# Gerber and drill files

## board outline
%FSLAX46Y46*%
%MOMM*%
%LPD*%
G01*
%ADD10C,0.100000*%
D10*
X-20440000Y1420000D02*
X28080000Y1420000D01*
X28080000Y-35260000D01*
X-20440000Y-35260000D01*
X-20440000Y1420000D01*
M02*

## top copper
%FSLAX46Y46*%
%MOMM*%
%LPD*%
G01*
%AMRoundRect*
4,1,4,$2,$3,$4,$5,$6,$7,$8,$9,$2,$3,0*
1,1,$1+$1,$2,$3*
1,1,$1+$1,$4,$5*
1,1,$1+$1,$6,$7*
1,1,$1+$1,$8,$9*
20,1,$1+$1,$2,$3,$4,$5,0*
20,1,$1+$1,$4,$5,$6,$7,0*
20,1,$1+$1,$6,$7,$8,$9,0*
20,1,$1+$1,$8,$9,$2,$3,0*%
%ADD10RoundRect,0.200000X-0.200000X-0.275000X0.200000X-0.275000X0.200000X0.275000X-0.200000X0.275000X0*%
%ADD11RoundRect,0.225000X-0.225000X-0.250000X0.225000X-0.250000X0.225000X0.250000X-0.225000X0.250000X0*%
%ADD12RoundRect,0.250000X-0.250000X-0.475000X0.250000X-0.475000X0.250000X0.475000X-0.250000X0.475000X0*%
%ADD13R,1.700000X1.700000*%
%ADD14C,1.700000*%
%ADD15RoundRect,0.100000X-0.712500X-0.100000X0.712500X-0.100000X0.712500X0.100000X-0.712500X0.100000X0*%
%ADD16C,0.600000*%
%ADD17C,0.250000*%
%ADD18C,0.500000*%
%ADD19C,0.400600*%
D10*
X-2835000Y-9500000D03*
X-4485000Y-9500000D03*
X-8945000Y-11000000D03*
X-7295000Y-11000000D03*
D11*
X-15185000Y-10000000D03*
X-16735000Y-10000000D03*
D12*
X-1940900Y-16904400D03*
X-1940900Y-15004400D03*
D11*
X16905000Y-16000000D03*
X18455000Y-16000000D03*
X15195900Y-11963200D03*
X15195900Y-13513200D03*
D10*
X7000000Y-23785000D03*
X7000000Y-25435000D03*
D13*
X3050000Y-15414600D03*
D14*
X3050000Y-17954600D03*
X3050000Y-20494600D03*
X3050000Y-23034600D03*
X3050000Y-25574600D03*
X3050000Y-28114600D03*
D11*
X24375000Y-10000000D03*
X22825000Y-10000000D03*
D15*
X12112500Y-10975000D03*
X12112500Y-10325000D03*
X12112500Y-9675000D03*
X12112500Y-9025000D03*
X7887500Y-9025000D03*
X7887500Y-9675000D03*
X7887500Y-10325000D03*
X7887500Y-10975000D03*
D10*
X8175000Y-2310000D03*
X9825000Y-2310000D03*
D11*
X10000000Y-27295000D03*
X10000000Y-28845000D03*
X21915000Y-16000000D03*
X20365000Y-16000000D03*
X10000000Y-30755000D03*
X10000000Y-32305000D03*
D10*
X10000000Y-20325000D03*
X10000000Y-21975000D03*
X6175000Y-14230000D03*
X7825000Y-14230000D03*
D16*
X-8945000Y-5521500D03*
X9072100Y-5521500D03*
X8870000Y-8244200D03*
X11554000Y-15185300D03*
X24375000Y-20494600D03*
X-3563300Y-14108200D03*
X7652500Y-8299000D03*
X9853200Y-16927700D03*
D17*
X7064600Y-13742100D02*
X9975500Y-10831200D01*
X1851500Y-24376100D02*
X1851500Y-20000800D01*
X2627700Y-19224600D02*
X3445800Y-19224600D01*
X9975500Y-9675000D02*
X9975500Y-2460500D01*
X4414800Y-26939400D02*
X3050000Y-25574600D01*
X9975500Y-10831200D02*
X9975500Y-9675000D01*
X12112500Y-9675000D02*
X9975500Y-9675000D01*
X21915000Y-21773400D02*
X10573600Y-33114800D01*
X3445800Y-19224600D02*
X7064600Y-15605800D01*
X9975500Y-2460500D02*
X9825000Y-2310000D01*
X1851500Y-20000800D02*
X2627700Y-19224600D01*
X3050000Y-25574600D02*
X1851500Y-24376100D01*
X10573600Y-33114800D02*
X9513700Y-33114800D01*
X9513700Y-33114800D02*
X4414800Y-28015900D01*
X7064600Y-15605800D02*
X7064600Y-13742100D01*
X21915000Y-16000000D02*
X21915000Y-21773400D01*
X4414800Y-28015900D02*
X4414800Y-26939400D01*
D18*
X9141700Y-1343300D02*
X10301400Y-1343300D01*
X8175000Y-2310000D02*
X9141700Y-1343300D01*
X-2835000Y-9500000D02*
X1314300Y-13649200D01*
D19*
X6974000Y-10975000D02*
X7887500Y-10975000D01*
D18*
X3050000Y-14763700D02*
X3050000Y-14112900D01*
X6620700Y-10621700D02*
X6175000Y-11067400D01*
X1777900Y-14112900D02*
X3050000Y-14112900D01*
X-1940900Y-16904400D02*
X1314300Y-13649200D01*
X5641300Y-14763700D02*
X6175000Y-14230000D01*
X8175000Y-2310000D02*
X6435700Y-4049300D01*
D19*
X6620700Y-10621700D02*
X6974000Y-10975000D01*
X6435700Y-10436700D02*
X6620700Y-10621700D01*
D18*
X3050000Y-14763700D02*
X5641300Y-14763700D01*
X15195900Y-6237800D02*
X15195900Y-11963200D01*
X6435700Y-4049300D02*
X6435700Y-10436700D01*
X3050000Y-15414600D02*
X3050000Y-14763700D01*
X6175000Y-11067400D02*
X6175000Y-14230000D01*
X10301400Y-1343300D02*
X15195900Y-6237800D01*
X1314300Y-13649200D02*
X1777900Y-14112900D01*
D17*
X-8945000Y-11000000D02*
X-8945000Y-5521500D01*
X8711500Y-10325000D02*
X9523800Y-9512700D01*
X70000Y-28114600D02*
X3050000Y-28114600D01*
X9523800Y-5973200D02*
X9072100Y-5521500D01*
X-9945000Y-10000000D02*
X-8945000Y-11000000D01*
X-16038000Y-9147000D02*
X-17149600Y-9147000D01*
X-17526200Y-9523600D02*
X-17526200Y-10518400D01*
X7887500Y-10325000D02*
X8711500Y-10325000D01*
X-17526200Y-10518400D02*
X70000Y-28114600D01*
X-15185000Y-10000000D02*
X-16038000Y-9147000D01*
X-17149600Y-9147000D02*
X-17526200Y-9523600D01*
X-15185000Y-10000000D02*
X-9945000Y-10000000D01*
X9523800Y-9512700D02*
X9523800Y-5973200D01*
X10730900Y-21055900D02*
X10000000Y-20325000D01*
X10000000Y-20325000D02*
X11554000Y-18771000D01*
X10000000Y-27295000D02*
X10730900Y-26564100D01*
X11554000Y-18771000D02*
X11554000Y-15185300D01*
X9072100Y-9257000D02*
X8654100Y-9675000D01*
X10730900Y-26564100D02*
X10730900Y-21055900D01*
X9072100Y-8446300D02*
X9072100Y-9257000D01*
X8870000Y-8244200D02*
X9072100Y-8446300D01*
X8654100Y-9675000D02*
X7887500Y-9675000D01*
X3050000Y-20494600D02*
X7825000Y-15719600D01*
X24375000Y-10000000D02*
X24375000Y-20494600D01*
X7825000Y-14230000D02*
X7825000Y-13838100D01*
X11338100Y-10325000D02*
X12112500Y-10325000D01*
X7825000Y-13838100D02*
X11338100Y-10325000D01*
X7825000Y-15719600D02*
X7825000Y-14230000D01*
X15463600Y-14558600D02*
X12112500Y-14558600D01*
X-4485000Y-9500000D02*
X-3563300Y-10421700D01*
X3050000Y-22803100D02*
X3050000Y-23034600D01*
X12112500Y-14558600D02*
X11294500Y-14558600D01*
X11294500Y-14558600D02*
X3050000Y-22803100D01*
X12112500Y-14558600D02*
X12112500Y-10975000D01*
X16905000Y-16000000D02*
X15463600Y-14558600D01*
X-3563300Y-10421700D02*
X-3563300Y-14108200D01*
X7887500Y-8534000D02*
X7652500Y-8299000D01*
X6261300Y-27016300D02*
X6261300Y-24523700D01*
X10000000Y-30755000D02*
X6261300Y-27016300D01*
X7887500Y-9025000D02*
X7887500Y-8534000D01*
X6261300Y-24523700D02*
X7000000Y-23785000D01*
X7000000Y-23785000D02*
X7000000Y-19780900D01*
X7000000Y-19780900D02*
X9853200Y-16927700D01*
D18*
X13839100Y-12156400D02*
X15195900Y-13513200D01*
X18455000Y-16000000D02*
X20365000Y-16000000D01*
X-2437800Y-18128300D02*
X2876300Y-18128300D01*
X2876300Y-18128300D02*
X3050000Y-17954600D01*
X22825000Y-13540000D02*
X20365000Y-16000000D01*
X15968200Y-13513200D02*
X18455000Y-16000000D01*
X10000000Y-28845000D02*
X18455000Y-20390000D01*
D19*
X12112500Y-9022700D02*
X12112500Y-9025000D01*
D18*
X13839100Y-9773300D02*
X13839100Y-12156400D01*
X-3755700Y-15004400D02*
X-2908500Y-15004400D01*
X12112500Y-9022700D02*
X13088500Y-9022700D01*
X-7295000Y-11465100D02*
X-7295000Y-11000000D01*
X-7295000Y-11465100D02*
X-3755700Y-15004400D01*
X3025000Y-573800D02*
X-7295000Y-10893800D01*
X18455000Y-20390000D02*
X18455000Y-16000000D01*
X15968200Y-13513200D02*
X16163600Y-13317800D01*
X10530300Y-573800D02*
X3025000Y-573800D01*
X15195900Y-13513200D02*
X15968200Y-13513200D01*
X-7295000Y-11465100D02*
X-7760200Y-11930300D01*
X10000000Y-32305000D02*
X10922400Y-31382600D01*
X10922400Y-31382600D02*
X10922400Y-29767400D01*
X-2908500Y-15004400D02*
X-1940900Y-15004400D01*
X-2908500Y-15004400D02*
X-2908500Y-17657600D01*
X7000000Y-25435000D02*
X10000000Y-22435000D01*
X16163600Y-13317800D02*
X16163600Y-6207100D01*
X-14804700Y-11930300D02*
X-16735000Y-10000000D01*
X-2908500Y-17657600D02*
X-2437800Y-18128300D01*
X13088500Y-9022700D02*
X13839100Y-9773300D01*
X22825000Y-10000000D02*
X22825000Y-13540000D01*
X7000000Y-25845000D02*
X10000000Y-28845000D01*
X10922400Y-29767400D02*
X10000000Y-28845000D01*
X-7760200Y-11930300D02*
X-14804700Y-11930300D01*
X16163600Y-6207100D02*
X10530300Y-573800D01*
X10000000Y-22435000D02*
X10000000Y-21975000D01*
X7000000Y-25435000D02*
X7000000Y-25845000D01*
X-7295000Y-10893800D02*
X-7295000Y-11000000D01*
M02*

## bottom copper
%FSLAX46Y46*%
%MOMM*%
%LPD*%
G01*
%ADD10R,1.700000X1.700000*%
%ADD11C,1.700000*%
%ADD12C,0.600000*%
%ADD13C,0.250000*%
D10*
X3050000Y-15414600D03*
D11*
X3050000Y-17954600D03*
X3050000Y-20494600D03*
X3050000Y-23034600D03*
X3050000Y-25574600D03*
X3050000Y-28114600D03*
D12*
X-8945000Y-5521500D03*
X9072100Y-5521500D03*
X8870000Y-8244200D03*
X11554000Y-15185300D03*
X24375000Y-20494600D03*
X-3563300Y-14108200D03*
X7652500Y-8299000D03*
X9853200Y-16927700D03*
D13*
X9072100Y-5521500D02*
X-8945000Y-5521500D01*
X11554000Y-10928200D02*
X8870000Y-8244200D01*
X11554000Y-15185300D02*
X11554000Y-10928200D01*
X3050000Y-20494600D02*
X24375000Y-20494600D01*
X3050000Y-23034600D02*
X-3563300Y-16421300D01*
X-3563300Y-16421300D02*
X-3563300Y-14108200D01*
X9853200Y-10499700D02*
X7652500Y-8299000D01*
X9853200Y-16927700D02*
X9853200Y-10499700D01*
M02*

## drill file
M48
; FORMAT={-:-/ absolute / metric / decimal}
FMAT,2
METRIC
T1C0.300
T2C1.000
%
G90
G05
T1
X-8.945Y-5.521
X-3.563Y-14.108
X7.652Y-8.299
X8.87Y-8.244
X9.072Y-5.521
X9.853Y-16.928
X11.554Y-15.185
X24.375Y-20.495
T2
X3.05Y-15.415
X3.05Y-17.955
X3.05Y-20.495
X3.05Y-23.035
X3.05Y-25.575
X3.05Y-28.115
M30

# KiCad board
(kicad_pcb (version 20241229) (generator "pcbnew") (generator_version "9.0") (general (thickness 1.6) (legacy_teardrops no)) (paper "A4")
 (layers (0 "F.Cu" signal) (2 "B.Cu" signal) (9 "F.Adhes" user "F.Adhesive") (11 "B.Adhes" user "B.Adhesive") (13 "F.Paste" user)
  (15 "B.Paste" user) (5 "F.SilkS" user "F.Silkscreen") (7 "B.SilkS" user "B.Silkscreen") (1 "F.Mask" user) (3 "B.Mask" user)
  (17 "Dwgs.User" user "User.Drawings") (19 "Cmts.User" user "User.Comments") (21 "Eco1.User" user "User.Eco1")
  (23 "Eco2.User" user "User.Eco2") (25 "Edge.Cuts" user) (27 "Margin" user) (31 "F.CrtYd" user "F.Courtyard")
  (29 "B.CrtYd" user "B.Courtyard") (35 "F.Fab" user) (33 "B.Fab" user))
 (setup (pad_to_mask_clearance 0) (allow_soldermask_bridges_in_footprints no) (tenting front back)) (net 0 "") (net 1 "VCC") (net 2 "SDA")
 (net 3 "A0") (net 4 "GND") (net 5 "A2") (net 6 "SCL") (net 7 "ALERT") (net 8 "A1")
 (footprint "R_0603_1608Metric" (layer "F.Cu") (at -3.66 9.5 180)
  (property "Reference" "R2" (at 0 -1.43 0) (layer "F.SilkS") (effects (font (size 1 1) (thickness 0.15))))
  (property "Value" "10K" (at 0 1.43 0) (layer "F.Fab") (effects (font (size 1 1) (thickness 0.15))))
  (pad "1" smd roundrect (at -0.825 0) (size 0.8 0.95) (layers "F.Cu" "F.Mask" "F.Paste") (roundrect_rratio 0.25) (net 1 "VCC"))
  (pad "2" smd roundrect (at 0.825 0) (size 0.8 0.95) (layers "F.Cu" "F.Mask" "F.Paste") (roundrect_rratio 0.25) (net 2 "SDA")))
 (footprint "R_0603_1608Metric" (layer "F.Cu") (at -8.12 11)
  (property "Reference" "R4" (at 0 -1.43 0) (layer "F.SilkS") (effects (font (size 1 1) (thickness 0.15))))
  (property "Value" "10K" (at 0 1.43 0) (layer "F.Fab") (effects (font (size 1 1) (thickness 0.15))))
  (pad "1" smd roundrect (at -0.825 0) (size 0.8 0.95) (layers "F.Cu" "F.Mask" "F.Paste") (roundrect_rratio 0.25) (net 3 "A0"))
  (pad "2" smd roundrect (at 0.825 0) (size 0.8 0.95) (layers "F.Cu" "F.Mask" "F.Paste") (roundrect_rratio 0.25) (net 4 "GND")))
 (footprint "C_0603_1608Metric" (layer "F.Cu") (at -15.96 10 180)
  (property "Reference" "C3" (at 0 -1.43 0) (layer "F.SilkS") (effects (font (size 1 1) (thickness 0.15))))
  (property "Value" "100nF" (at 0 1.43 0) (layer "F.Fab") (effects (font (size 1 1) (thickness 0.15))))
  (pad "1" smd roundrect (at -0.775 0) (size 0.9 0.95) (layers "F.Cu" "F.Mask" "F.Paste") (roundrect_rratio 0.25) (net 3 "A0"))
  (pad "2" smd roundrect (at 0.775 0) (size 0.9 0.95) (layers "F.Cu" "F.Mask" "F.Paste") (roundrect_rratio 0.25) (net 4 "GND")))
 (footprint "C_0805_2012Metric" (layer "F.Cu") (at -1.9409 15.9544 90)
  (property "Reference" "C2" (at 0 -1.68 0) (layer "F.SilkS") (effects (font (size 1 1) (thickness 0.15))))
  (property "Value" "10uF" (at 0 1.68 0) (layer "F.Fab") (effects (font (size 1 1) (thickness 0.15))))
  (pad "1" smd roundrect (at -0.95 0) (size 1 1.45) (layers "F.Cu" "F.Mask" "F.Paste") (roundrect_rratio 0.25) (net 1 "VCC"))
  (pad "2" smd roundrect (at 0.95 0) (size 1 1.45) (layers "F.Cu" "F.Mask" "F.Paste") (roundrect_rratio 0.25) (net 4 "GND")))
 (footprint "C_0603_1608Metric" (layer "F.Cu") (at 17.68 16)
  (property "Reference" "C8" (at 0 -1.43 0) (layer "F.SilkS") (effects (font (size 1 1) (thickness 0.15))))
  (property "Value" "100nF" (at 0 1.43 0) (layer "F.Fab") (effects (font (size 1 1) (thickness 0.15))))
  (pad "1" smd roundrect (at -0.775 0) (size 0.9 0.95) (layers "F.Cu" "F.Mask" "F.Paste") (roundrect_rratio 0.25) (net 2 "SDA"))
  (pad "2" smd roundrect (at 0.775 0) (size 0.9 0.95) (layers "F.Cu" "F.Mask" "F.Paste") (roundrect_rratio 0.25) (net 4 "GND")))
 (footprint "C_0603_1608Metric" (layer "F.Cu") (at 15.1959 12.7382 -90)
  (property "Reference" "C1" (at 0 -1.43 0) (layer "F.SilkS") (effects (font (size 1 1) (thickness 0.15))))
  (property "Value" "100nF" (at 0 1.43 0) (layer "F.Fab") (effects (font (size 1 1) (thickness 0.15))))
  (pad "1" smd roundrect (at -0.775 0) (size 0.9 0.95) (layers "F.Cu" "F.Mask" "F.Paste") (roundrect_rratio 0.25) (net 1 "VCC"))
  (pad "2" smd roundrect (at 0.775 0) (size 0.9 0.95) (layers "F.Cu" "F.Mask" "F.Paste") (roundrect_rratio 0.25) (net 4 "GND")))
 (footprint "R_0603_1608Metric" (layer "F.Cu") (at 7 24.61 -90)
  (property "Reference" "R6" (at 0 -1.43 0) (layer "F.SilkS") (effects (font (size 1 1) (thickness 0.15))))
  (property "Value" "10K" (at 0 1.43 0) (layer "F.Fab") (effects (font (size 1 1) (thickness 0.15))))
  (pad "1" smd roundrect (at -0.825 0) (size 0.8 0.95) (layers "F.Cu" "F.Mask" "F.Paste") (roundrect_rratio 0.25) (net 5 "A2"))
  (pad "2" smd roundrect (at 0.825 0) (size 0.8 0.95) (layers "F.Cu" "F.Mask" "F.Paste") (roundrect_rratio 0.25) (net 4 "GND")))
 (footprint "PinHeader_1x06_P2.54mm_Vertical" (layer "F.Cu") (at 3.05 15.4146)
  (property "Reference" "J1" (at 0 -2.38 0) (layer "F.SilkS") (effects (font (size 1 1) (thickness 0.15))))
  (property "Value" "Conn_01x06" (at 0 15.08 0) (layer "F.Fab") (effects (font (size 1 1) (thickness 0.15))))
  (pad "1" thru_hole rect (at 0 0) (size 1.7 1.7) (drill 1) (layers "*.Cu" "*.Mask") (remove_unused_layers no) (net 1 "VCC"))
  (pad "2" thru_hole circle (at 0 2.54) (size 1.7 1.7) (drill 1) (layers "*.Cu" "*.Mask") (remove_unused_layers no) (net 4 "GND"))
  (pad "3" thru_hole circle (at 0 5.08) (size 1.7 1.7) (drill 1) (layers "*.Cu" "*.Mask") (remove_unused_layers no) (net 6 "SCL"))
  (pad "4" thru_hole circle (at 0 7.62) (size 1.7 1.7) (drill 1) (layers "*.Cu" "*.Mask") (remove_unused_layers no) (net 2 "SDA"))
  (pad "5" thru_hole circle (at 0 10.16) (size 1.7 1.7) (drill 1) (layers "*.Cu" "*.Mask") (remove_unused_layers no) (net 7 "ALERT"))
  (pad "6" thru_hole circle (at 0 12.7) (size 1.7 1.7) (drill 1) (layers "*.Cu" "*.Mask") (remove_unused_layers no) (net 3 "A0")))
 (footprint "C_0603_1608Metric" (layer "F.Cu") (at 23.6 10 180)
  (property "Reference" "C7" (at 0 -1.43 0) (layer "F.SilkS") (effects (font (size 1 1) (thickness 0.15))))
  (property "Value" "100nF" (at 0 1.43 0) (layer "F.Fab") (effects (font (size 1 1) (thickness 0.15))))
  (pad "1" smd roundrect (at -0.775 0) (size 0.9 0.95) (layers "F.Cu" "F.Mask" "F.Paste") (roundrect_rratio 0.25) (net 6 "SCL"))
  (pad "2" smd roundrect (at 0.775 0) (size 0.9 0.95) (layers "F.Cu" "F.Mask" "F.Paste") (roundrect_rratio 0.25) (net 4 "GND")))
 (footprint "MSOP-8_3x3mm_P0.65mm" (layer "F.Cu") (at 10 10 180)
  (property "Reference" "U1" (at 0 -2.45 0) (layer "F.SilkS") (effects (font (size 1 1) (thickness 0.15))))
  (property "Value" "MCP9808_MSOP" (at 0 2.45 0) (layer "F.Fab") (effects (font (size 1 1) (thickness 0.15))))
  (pad "1" smd roundrect (at -2.1125 -0.975) (size 1.625 0.4) (layers "F.Cu" "F.Mask" "F.Paste") (roundrect_rratio 0.25) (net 2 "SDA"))
  (pad "2" smd roundrect (at -2.1125 -0.325) (size 1.625 0.4) (layers "F.Cu" "F.Mask" "F.Paste") (roundrect_rratio 0.25) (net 6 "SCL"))
  (pad "3" smd roundrect (at -2.1125 0.325) (size 1.625 0.4) (layers "F.Cu" "F.Mask" "F.Paste") (roundrect_rratio 0.25) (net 7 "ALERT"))
  (pad "4" smd roundrect (at -2.1125 0.975) (size 1.625 0.4) (layers "F.Cu" "F.Mask" "F.Paste") (roundrect_rratio 0.25) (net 4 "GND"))
  (pad "5" smd roundrect (at 2.1125 0.975) (size 1.625 0.4) (layers "F.Cu" "F.Mask" "F.Paste") (roundrect_rratio 0.25) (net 5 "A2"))
  (pad "6" smd roundrect (at 2.1125 0.325) (size 1.625 0.4) (layers "F.Cu" "F.Mask" "F.Paste") (roundrect_rratio 0.25) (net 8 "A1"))
  (pad "7" smd roundrect (at 2.1125 -0.325) (size 1.625 0.4) (layers "F.Cu" "F.Mask" "F.Paste") (roundrect_rratio 0.25) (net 3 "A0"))
  (pad "8" smd roundrect (at 2.1125 -0.975) (size 1.625 0.4) (layers "F.Cu" "F.Mask" "F.Paste") (roundrect_rratio 0.25) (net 1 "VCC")))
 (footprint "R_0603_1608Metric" (layer "F.Cu") (at 9 2.31)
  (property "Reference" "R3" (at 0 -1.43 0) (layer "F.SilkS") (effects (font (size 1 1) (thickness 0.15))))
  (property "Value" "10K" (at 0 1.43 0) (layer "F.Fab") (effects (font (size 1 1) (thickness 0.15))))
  (pad "1" smd roundrect (at -0.825 0) (size 0.8 0.95) (layers "F.Cu" "F.Mask" "F.Paste") (roundrect_rratio 0.25) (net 1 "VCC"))
  (pad "2" smd roundrect (at 0.825 0) (size 0.8 0.95) (layers "F.Cu" "F.Mask" "F.Paste") (roundrect_rratio 0.25) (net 7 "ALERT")))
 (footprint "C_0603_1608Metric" (layer "F.Cu") (at 10 28.07 -90)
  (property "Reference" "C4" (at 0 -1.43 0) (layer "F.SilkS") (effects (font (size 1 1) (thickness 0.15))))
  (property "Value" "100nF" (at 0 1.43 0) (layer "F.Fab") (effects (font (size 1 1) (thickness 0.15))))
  (pad "1" smd roundrect (at -0.775 0) (size 0.9 0.95) (layers "F.Cu" "F.Mask" "F.Paste") (roundrect_rratio 0.25) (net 8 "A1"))
  (pad "2" smd roundrect (at 0.775 0) (size 0.9 0.95) (layers "F.Cu" "F.Mask" "F.Paste") (roundrect_rratio 0.25) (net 4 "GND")))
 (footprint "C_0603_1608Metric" (layer "F.Cu") (at 21.14 16 180)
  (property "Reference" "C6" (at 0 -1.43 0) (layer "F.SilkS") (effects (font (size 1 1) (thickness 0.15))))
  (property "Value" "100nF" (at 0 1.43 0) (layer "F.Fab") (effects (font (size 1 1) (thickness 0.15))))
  (pad "1" smd roundrect (at -0.775 0) (size 0.9 0.95) (layers "F.Cu" "F.Mask" "F.Paste") (roundrect_rratio 0.25) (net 7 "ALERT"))
  (pad "2" smd roundrect (at 0.775 0) (size 0.9 0.95) (layers "F.Cu" "F.Mask" "F.Paste") (roundrect_rratio 0.25) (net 4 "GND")))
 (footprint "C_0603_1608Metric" (layer "F.Cu") (at 10 31.53 -90)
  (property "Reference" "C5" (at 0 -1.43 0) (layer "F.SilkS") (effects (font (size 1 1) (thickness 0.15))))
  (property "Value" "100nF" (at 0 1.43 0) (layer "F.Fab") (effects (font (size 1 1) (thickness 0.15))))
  (pad "1" smd roundrect (at -0.775 0) (size 0.9 0.95) (layers "F.Cu" "F.Mask" "F.Paste") (roundrect_rratio 0.25) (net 5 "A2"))
  (pad "2" smd roundrect (at 0.775 0) (size 0.9 0.95) (layers "F.Cu" "F.Mask" "F.Paste") (roundrect_rratio 0.25) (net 4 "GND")))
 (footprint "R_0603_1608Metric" (layer "F.Cu") (at 10 21.15 -90)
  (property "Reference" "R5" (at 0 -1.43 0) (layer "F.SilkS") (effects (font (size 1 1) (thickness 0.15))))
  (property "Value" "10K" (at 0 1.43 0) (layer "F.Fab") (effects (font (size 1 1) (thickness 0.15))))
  (pad "1" smd roundrect (at -0.825 0) (size 0.8 0.95) (layers "F.Cu" "F.Mask" "F.Paste") (roundrect_rratio 0.25) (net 8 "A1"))
  (pad "2" smd roundrect (at 0.825 0) (size 0.8 0.95) (layers "F.Cu" "F.Mask" "F.Paste") (roundrect_rratio 0.25) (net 4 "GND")))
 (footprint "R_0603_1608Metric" (layer "F.Cu") (at 7 14.23)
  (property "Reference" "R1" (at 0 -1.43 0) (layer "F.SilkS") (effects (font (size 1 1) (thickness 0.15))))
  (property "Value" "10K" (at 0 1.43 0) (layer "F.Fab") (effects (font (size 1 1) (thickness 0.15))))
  (pad "1" smd roundrect (at -0.825 0) (size 0.8 0.95) (layers "F.Cu" "F.Mask" "F.Paste") (roundrect_rratio 0.25) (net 1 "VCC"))
  (pad "2" smd roundrect (at 0.825 0) (size 0.8 0.95) (layers "F.Cu" "F.Mask" "F.Paste") (roundrect_rratio 0.25) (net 6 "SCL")))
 (gr_rect (start -20.44 -1.42) (end 28.08 35.26) (stroke (width 0.1) (type solid)) (fill no) (layer "Edge.Cuts"))
 (segment (start 7.0646 13.7421) (end 9.9755 10.8312) (width 0.25) (layer "F.Cu") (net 7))
 (segment (start 1.8515 24.3761) (end 1.8515 20.0008) (width 0.25) (layer "F.Cu") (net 7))
 (segment (start 2.6277 19.2246) (end 3.4458 19.2246) (width 0.25) (layer "F.Cu") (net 7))
 (segment (start 9.9755 9.675) (end 9.9755 2.4605) (width 0.25) (layer "F.Cu") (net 7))
 (segment (start 4.4148 26.9394) (end 3.05 25.5746) (width 0.25) (layer "F.Cu") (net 7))
 (segment (start 9.9755 10.8312) (end 9.9755 9.675) (width 0.25) (layer "F.Cu") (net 7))
 (segment (start 12.1125 9.675) (end 9.9755 9.675) (width 0.25) (layer "F.Cu") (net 7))
 (segment (start 21.915 21.7734) (end 10.5736 33.1148) (width 0.25) (layer "F.Cu") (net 7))
 (segment (start 3.4458 19.2246) (end 7.0646 15.6058) (width 0.25) (layer "F.Cu") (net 7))
 (segment (start 9.9755 2.4605) (end 9.825 2.31) (width 0.25) (layer "F.Cu") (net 7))
 (segment (start 1.8515 20.0008) (end 2.6277 19.2246) (width 0.25) (layer "F.Cu") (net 7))
 (segment (start 3.05 25.5746) (end 1.8515 24.3761) (width 0.25) (layer "F.Cu") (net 7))
 (segment (start 10.5736 33.1148) (end 9.5137 33.1148) (width 0.25) (layer "F.Cu") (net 7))
 (segment (start 9.5137 33.1148) (end 4.4148 28.0159) (width 0.25) (layer "F.Cu") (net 7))
 (segment (start 7.0646 15.6058) (end 7.0646 13.7421) (width 0.25) (layer "F.Cu") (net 7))
 (segment (start 21.915 16) (end 21.915 21.7734) (width 0.25) (layer "F.Cu") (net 7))
 (segment (start 4.4148 28.0159) (end 4.4148 26.9394) (width 0.25) (layer "F.Cu") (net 7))
 (segment (start 9.1417 1.3433) (end 10.3014 1.3433) (width 0.5) (layer "F.Cu") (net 1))
 (segment (start 8.175 2.31) (end 9.1417 1.3433) (width 0.5) (layer "F.Cu") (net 1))
 (segment (start -2.835 9.5) (end 1.3143 13.6492) (width 0.5) (layer "F.Cu") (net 1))
 (segment (start 6.974 10.975) (end 7.8875 10.975) (width 0.4006) (layer "F.Cu") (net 1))
 (segment (start 3.05 14.7637) (end 3.05 14.1129) (width 0.5) (layer "F.Cu") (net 1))
 (segment (start 6.6207 10.6217) (end 6.175 11.0674) (width 0.5) (layer "F.Cu") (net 1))
 (segment (start 1.7779 14.1129) (end 3.05 14.1129) (width 0.5) (layer "F.Cu") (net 1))
 (segment (start -1.9409 16.9044) (end 1.3143 13.6492) (width 0.5) (layer "F.Cu") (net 1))
 (segment (start 5.6413 14.7637) (end 6.175 14.23) (width 0.5) (layer "F.Cu") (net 1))
 (segment (start 8.175 2.31) (end 6.4357 4.0493) (width 0.5) (layer "F.Cu") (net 1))
 (segment (start 6.6207 10.6217) (end 6.974 10.975) (width 0.4006) (layer "F.Cu") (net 1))
 (segment (start 6.4357 10.4367) (end 6.6207 10.6217) (width 0.4006) (layer "F.Cu") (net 1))
 (segment (start 3.05 14.7637) (end 5.6413 14.7637) (width 0.5) (layer "F.Cu") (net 1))
 (segment (start 15.1959 6.2378) (end 15.1959 11.9632) (width 0.5) (layer "F.Cu") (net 1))
 (segment (start 6.4357 4.0493) (end 6.4357 10.4367) (width 0.5) (layer "F.Cu") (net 1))
 (segment (start 3.05 15.4146) (end 3.05 14.7637) (width 0.5) (layer "F.Cu") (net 1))
 (segment (start 6.175 11.0674) (end 6.175 14.23) (width 0.5) (layer "F.Cu") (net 1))
 (segment (start 10.3014 1.3433) (end 15.1959 6.2378) (width 0.5) (layer "F.Cu") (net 1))
 (segment (start 1.3143 13.6492) (end 1.7779 14.1129) (width 0.5) (layer "F.Cu") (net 1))
 (segment (start -8.945 11) (end -8.945 5.5215) (width 0.25) (layer "F.Cu") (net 3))
 (segment (start 8.7115 10.325) (end 9.5238 9.5127) (width 0.25) (layer "F.Cu") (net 3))
 (segment (start 0.07 28.1146) (end 3.05 28.1146) (width 0.25) (layer "F.Cu") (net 3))
 (segment (start 9.5238 5.9732) (end 9.0721 5.5215) (width 0.25) (layer "F.Cu") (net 3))
 (segment (start -9.945 10) (end -8.945 11) (width 0.25) (layer "F.Cu") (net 3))
 (segment (start -16.038 9.147) (end -17.1496 9.147) (width 0.25) (layer "F.Cu") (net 3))
 (segment (start -17.5262 9.5236) (end -17.5262 10.5184) (width 0.25) (layer "F.Cu") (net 3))
 (segment (start 7.8875 10.325) (end 8.7115 10.325) (width 0.25) (layer "F.Cu") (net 3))
 (segment (start -17.5262 10.5184) (end 0.07 28.1146) (width 0.25) (layer "F.Cu") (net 3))
 (segment (start -15.185 10) (end -16.038 9.147) (width 0.25) (layer "F.Cu") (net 3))
 (segment (start -17.1496 9.147) (end -17.5262 9.5236) (width 0.25) (layer "F.Cu") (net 3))
 (segment (start -15.185 10) (end -9.945 10) (width 0.25) (layer "F.Cu") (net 3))
 (segment (start 9.5238 9.5127) (end 9.5238 5.9732) (width 0.25) (layer "F.Cu") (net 3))
 (via (at -8.945 5.5215) (size 0.6) (drill 0.3) (layers "F.Cu" "B.Cu") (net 3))
 (via (at 9.0721 5.5215) (size 0.6) (drill 0.3) (layers "F.Cu" "B.Cu") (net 3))
 (segment (start 9.0721 5.5215) (end -8.945 5.5215) (width 0.25) (layer "B.Cu") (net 3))
 (segment (start 10.7309 21.0559) (end 10 20.325) (width 0.25) (layer "F.Cu") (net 8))
 (segment (start 10 20.325) (end 11.554 18.771) (width 0.25) (layer "F.Cu") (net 8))
 (segment (start 10 27.295) (end 10.7309 26.5641) (width 0.25) (layer "F.Cu") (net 8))
 (segment (start 11.554 18.771) (end 11.554 15.1853) (width 0.25) (layer "F.Cu") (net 8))
 (segment (start 9.0721 9.257) (end 8.6541 9.675) (width 0.25) (layer "F.Cu") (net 8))
 (segment (start 10.7309 26.5641) (end 10.7309 21.0559) (width 0.25) (layer "F.Cu") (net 8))
 (segment (start 9.0721 8.4463) (end 9.0721 9.257) (width 0.25) (layer "F.Cu") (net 8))
 (segment (start 8.87 8.2442) (end 9.0721 8.4463) (width 0.25) (layer "F.Cu") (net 8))
 (segment (start 8.6541 9.675) (end 7.8875 9.675) (width 0.25) (layer "F.Cu") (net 8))
 (via (at 8.87 8.2442) (size 0.6) (drill 0.3) (layers "F.Cu" "B.Cu") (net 8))
 (via (at 11.554 15.1853) (size 0.6) (drill 0.3) (layers "F.Cu" "B.Cu") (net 8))
 (segment (start 11.554 10.9282) (end 8.87 8.2442) (width 0.25) (layer "B.Cu") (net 8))
 (segment (start 11.554 15.1853) (end 11.554 10.9282) (width 0.25) (layer "B.Cu") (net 8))
 (segment (start 3.05 20.4946) (end 7.825 15.7196) (width 0.25) (layer "F.Cu") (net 6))
 (segment (start 24.375 10) (end 24.375 20.4946) (width 0.25) (layer "F.Cu") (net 6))
 (segment (start 7.825 14.23) (end 7.825 13.8381) (width 0.25) (layer "F.Cu") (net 6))
 (segment (start 11.3381 10.325) (end 12.1125 10.325) (width 0.25) (layer "F.Cu") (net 6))
 (segment (start 7.825 13.8381) (end 11.3381 10.325) (width 0.25) (layer "F.Cu") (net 6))
 (segment (start 7.825 15.7196) (end 7.825 14.23) (width 0.25) (layer "F.Cu") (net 6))
 (via (at 24.375 20.4946) (size 0.6) (drill 0.3) (layers "F.Cu" "B.Cu") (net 6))
 (segment (start 3.05 20.4946) (end 24.375 20.4946) (width 0.25) (layer "B.Cu") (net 6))
 (segment (start 15.4636 14.5586) (end 12.1125 14.5586) (width 0.25) (layer "F.Cu") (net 2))
 (segment (start -4.485 9.5) (end -3.5633 10.4217) (width 0.25) (layer "F.Cu") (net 2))
 (segment (start 3.05 22.8031) (end 3.05 23.0346) (width 0.25) (layer "F.Cu") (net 2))
 (segment (start 12.1125 14.5586) (end 11.2945 14.5586) (width 0.25) (layer "F.Cu") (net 2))
 (segment (start 11.2945 14.5586) (end 3.05 22.8031) (width 0.25) (layer "F.Cu") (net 2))
 (segment (start 12.1125 14.5586) (end 12.1125 10.975) (width 0.25) (layer "F.Cu") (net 2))
 (segment (start 16.905 16) (end 15.4636 14.5586) (width 0.25) (layer "F.Cu") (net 2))
 (segment (start -3.5633 10.4217) (end -3.5633 14.1082) (width 0.25) (layer "F.Cu") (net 2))
 (via (at -3.5633 14.1082) (size 0.6) (drill 0.3) (layers "F.Cu" "B.Cu") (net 2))
 (segment (start 3.05 23.0346) (end -3.5633 16.4213) (width 0.25) (layer "B.Cu") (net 2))
 (segment (start -3.5633 16.4213) (end -3.5633 14.1082) (width 0.25) (layer "B.Cu") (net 2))
 (segment (start 7.8875 8.534) (end 7.6525 8.299) (width 0.25) (layer "F.Cu") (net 5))
 (segment (start 6.2613 27.0163) (end 6.2613 24.5237) (width 0.25) (layer "F.Cu") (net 5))
 (segment (start 10 30.755) (end 6.2613 27.0163) (width 0.25) (layer "F.Cu") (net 5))
 (segment (start 7.8875 9.025) (end 7.8875 8.534) (width 0.25) (layer "F.Cu") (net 5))
 (segment (start 6.2613 24.5237) (end 7 23.785) (width 0.25) (layer "F.Cu") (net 5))
 (segment (start 7 23.785) (end 7 19.7809) (width 0.25) (layer "F.Cu") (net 5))
 (segment (start 7 19.7809) (end 9.8532 16.9277) (width 0.25) (layer "F.Cu") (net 5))
 (via (at 7.6525 8.299) (size 0.6) (drill 0.3) (layers "F.Cu" "B.Cu") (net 5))
 (via (at 9.8532 16.9277) (size 0.6) (drill 0.3) (layers "F.Cu" "B.Cu") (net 5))
 (segment (start 9.8532 10.4997) (end 7.6525 8.299) (width 0.25) (layer "B.Cu") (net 5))
 (segment (start 9.8532 16.9277) (end 9.8532 10.4997) (width 0.25) (layer "B.Cu") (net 5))
 (segment (start 13.8391 12.1564) (end 15.1959 13.5132) (width 0.5) (layer "F.Cu") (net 4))
 (segment (start 18.455 16) (end 20.365 16) (width 0.5) (layer "F.Cu") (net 4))
 (segment (start -2.4378 18.1283) (end 2.8763 18.1283) (width 0.5) (layer "F.Cu") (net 4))
 (segment (start 2.8763 18.1283) (end 3.05 17.9546) (width 0.5) (layer "F.Cu") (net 4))
 (segment (start 22.825 13.54) (end 20.365 16) (width 0.5) (layer "F.Cu") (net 4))
 (segment (start 15.9682 13.5132) (end 18.455 16) (width 0.5) (layer "F.Cu") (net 4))
 (segment (start 10 28.845) (end 18.455 20.39) (width 0.5) (layer "F.Cu") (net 4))
 (segment (start 12.1125 9.0227) (end 12.1125 9.025) (width 0.4006) (layer "F.Cu") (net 4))
 (segment (start 13.8391 9.7733) (end 13.8391 12.1564) (width 0.5) (layer "F.Cu") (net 4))
 (segment (start -3.7557 15.0044) (end -2.9085 15.0044) (width 0.5) (layer "F.Cu") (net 4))
 (segment (start 12.1125 9.0227) (end 13.0885 9.0227) (width 0.5) (layer "F.Cu") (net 4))
 (segment (start -7.295 11.4651) (end -7.295 11) (width 0.5) (layer "F.Cu") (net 4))
 (segment (start -7.295 11.4651) (end -3.7557 15.0044) (width 0.5) (layer "F.Cu") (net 4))
 (segment (start 3.025 0.5738) (end -7.295 10.8938) (width 0.5) (layer "F.Cu") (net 4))
 (segment (start 18.455 20.39) (end 18.455 16) (width 0.5) (layer "F.Cu") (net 4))
 (segment (start 15.9682 13.5132) (end 16.1636 13.3178) (width 0.5) (layer "F.Cu") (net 4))
 (segment (start 10.5303 0.5738) (end 3.025 0.5738) (width 0.5) (layer "F.Cu") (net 4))
 (segment (start 15.1959 13.5132) (end 15.9682 13.5132) (width 0.5) (layer "F.Cu") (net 4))
 (segment (start -7.295 11.4651) (end -7.7602 11.9303) (width 0.5) (layer "F.Cu") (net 4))
 (segment (start 10 32.305) (end 10.9224 31.3826) (width 0.5) (layer "F.Cu") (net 4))
 (segment (start 10.9224 31.3826) (end 10.9224 29.7674) (width 0.5) (layer "F.Cu") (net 4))
 (segment (start -2.9085 15.0044) (end -1.9409 15.0044) (width 0.5) (layer "F.Cu") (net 4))
 (segment (start -2.9085 15.0044) (end -2.9085 17.6576) (width 0.5) (layer "F.Cu") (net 4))
 (segment (start 7 25.435) (end 10 22.435) (width 0.5) (layer "F.Cu") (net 4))
 (segment (start 16.1636 13.3178) (end 16.1636 6.2071) (width 0.5) (layer "F.Cu") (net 4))
 (segment (start -14.8047 11.9303) (end -16.735 10) (width 0.5) (layer "F.Cu") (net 4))
 (segment (start -2.9085 17.6576) (end -2.4378 18.1283) (width 0.5) (layer "F.Cu") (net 4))
 (segment (start 13.0885 9.0227) (end 13.8391 9.7733) (width 0.5) (layer "F.Cu") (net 4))
 (segment (start 22.825 10) (end 22.825 13.54) (width 0.5) (layer "F.Cu") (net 4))
 (segment (start 7 25.845) (end 10 28.845) (width 0.5) (layer "F.Cu") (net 4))
 (segment (start 10.9224 29.7674) (end 10 28.845) (width 0.5) (layer "F.Cu") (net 4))
 (segment (start -7.7602 11.9303) (end -14.8047 11.9303) (width 0.5) (layer "F.Cu") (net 4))
 (segment (start 16.1636 6.2071) (end 10.5303 0.5738) (width 0.5) (layer "F.Cu") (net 4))
 (segment (start 10 22.435) (end 10 21.975) (width 0.5) (layer "F.Cu") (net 4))
 (segment (start 7 25.435) (end 7 25.845) (width 0.5) (layer "F.Cu") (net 4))
 (segment (start -7.295 10.8938) (end -7.295 11) (width 0.5) (layer "F.Cu") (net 4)))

